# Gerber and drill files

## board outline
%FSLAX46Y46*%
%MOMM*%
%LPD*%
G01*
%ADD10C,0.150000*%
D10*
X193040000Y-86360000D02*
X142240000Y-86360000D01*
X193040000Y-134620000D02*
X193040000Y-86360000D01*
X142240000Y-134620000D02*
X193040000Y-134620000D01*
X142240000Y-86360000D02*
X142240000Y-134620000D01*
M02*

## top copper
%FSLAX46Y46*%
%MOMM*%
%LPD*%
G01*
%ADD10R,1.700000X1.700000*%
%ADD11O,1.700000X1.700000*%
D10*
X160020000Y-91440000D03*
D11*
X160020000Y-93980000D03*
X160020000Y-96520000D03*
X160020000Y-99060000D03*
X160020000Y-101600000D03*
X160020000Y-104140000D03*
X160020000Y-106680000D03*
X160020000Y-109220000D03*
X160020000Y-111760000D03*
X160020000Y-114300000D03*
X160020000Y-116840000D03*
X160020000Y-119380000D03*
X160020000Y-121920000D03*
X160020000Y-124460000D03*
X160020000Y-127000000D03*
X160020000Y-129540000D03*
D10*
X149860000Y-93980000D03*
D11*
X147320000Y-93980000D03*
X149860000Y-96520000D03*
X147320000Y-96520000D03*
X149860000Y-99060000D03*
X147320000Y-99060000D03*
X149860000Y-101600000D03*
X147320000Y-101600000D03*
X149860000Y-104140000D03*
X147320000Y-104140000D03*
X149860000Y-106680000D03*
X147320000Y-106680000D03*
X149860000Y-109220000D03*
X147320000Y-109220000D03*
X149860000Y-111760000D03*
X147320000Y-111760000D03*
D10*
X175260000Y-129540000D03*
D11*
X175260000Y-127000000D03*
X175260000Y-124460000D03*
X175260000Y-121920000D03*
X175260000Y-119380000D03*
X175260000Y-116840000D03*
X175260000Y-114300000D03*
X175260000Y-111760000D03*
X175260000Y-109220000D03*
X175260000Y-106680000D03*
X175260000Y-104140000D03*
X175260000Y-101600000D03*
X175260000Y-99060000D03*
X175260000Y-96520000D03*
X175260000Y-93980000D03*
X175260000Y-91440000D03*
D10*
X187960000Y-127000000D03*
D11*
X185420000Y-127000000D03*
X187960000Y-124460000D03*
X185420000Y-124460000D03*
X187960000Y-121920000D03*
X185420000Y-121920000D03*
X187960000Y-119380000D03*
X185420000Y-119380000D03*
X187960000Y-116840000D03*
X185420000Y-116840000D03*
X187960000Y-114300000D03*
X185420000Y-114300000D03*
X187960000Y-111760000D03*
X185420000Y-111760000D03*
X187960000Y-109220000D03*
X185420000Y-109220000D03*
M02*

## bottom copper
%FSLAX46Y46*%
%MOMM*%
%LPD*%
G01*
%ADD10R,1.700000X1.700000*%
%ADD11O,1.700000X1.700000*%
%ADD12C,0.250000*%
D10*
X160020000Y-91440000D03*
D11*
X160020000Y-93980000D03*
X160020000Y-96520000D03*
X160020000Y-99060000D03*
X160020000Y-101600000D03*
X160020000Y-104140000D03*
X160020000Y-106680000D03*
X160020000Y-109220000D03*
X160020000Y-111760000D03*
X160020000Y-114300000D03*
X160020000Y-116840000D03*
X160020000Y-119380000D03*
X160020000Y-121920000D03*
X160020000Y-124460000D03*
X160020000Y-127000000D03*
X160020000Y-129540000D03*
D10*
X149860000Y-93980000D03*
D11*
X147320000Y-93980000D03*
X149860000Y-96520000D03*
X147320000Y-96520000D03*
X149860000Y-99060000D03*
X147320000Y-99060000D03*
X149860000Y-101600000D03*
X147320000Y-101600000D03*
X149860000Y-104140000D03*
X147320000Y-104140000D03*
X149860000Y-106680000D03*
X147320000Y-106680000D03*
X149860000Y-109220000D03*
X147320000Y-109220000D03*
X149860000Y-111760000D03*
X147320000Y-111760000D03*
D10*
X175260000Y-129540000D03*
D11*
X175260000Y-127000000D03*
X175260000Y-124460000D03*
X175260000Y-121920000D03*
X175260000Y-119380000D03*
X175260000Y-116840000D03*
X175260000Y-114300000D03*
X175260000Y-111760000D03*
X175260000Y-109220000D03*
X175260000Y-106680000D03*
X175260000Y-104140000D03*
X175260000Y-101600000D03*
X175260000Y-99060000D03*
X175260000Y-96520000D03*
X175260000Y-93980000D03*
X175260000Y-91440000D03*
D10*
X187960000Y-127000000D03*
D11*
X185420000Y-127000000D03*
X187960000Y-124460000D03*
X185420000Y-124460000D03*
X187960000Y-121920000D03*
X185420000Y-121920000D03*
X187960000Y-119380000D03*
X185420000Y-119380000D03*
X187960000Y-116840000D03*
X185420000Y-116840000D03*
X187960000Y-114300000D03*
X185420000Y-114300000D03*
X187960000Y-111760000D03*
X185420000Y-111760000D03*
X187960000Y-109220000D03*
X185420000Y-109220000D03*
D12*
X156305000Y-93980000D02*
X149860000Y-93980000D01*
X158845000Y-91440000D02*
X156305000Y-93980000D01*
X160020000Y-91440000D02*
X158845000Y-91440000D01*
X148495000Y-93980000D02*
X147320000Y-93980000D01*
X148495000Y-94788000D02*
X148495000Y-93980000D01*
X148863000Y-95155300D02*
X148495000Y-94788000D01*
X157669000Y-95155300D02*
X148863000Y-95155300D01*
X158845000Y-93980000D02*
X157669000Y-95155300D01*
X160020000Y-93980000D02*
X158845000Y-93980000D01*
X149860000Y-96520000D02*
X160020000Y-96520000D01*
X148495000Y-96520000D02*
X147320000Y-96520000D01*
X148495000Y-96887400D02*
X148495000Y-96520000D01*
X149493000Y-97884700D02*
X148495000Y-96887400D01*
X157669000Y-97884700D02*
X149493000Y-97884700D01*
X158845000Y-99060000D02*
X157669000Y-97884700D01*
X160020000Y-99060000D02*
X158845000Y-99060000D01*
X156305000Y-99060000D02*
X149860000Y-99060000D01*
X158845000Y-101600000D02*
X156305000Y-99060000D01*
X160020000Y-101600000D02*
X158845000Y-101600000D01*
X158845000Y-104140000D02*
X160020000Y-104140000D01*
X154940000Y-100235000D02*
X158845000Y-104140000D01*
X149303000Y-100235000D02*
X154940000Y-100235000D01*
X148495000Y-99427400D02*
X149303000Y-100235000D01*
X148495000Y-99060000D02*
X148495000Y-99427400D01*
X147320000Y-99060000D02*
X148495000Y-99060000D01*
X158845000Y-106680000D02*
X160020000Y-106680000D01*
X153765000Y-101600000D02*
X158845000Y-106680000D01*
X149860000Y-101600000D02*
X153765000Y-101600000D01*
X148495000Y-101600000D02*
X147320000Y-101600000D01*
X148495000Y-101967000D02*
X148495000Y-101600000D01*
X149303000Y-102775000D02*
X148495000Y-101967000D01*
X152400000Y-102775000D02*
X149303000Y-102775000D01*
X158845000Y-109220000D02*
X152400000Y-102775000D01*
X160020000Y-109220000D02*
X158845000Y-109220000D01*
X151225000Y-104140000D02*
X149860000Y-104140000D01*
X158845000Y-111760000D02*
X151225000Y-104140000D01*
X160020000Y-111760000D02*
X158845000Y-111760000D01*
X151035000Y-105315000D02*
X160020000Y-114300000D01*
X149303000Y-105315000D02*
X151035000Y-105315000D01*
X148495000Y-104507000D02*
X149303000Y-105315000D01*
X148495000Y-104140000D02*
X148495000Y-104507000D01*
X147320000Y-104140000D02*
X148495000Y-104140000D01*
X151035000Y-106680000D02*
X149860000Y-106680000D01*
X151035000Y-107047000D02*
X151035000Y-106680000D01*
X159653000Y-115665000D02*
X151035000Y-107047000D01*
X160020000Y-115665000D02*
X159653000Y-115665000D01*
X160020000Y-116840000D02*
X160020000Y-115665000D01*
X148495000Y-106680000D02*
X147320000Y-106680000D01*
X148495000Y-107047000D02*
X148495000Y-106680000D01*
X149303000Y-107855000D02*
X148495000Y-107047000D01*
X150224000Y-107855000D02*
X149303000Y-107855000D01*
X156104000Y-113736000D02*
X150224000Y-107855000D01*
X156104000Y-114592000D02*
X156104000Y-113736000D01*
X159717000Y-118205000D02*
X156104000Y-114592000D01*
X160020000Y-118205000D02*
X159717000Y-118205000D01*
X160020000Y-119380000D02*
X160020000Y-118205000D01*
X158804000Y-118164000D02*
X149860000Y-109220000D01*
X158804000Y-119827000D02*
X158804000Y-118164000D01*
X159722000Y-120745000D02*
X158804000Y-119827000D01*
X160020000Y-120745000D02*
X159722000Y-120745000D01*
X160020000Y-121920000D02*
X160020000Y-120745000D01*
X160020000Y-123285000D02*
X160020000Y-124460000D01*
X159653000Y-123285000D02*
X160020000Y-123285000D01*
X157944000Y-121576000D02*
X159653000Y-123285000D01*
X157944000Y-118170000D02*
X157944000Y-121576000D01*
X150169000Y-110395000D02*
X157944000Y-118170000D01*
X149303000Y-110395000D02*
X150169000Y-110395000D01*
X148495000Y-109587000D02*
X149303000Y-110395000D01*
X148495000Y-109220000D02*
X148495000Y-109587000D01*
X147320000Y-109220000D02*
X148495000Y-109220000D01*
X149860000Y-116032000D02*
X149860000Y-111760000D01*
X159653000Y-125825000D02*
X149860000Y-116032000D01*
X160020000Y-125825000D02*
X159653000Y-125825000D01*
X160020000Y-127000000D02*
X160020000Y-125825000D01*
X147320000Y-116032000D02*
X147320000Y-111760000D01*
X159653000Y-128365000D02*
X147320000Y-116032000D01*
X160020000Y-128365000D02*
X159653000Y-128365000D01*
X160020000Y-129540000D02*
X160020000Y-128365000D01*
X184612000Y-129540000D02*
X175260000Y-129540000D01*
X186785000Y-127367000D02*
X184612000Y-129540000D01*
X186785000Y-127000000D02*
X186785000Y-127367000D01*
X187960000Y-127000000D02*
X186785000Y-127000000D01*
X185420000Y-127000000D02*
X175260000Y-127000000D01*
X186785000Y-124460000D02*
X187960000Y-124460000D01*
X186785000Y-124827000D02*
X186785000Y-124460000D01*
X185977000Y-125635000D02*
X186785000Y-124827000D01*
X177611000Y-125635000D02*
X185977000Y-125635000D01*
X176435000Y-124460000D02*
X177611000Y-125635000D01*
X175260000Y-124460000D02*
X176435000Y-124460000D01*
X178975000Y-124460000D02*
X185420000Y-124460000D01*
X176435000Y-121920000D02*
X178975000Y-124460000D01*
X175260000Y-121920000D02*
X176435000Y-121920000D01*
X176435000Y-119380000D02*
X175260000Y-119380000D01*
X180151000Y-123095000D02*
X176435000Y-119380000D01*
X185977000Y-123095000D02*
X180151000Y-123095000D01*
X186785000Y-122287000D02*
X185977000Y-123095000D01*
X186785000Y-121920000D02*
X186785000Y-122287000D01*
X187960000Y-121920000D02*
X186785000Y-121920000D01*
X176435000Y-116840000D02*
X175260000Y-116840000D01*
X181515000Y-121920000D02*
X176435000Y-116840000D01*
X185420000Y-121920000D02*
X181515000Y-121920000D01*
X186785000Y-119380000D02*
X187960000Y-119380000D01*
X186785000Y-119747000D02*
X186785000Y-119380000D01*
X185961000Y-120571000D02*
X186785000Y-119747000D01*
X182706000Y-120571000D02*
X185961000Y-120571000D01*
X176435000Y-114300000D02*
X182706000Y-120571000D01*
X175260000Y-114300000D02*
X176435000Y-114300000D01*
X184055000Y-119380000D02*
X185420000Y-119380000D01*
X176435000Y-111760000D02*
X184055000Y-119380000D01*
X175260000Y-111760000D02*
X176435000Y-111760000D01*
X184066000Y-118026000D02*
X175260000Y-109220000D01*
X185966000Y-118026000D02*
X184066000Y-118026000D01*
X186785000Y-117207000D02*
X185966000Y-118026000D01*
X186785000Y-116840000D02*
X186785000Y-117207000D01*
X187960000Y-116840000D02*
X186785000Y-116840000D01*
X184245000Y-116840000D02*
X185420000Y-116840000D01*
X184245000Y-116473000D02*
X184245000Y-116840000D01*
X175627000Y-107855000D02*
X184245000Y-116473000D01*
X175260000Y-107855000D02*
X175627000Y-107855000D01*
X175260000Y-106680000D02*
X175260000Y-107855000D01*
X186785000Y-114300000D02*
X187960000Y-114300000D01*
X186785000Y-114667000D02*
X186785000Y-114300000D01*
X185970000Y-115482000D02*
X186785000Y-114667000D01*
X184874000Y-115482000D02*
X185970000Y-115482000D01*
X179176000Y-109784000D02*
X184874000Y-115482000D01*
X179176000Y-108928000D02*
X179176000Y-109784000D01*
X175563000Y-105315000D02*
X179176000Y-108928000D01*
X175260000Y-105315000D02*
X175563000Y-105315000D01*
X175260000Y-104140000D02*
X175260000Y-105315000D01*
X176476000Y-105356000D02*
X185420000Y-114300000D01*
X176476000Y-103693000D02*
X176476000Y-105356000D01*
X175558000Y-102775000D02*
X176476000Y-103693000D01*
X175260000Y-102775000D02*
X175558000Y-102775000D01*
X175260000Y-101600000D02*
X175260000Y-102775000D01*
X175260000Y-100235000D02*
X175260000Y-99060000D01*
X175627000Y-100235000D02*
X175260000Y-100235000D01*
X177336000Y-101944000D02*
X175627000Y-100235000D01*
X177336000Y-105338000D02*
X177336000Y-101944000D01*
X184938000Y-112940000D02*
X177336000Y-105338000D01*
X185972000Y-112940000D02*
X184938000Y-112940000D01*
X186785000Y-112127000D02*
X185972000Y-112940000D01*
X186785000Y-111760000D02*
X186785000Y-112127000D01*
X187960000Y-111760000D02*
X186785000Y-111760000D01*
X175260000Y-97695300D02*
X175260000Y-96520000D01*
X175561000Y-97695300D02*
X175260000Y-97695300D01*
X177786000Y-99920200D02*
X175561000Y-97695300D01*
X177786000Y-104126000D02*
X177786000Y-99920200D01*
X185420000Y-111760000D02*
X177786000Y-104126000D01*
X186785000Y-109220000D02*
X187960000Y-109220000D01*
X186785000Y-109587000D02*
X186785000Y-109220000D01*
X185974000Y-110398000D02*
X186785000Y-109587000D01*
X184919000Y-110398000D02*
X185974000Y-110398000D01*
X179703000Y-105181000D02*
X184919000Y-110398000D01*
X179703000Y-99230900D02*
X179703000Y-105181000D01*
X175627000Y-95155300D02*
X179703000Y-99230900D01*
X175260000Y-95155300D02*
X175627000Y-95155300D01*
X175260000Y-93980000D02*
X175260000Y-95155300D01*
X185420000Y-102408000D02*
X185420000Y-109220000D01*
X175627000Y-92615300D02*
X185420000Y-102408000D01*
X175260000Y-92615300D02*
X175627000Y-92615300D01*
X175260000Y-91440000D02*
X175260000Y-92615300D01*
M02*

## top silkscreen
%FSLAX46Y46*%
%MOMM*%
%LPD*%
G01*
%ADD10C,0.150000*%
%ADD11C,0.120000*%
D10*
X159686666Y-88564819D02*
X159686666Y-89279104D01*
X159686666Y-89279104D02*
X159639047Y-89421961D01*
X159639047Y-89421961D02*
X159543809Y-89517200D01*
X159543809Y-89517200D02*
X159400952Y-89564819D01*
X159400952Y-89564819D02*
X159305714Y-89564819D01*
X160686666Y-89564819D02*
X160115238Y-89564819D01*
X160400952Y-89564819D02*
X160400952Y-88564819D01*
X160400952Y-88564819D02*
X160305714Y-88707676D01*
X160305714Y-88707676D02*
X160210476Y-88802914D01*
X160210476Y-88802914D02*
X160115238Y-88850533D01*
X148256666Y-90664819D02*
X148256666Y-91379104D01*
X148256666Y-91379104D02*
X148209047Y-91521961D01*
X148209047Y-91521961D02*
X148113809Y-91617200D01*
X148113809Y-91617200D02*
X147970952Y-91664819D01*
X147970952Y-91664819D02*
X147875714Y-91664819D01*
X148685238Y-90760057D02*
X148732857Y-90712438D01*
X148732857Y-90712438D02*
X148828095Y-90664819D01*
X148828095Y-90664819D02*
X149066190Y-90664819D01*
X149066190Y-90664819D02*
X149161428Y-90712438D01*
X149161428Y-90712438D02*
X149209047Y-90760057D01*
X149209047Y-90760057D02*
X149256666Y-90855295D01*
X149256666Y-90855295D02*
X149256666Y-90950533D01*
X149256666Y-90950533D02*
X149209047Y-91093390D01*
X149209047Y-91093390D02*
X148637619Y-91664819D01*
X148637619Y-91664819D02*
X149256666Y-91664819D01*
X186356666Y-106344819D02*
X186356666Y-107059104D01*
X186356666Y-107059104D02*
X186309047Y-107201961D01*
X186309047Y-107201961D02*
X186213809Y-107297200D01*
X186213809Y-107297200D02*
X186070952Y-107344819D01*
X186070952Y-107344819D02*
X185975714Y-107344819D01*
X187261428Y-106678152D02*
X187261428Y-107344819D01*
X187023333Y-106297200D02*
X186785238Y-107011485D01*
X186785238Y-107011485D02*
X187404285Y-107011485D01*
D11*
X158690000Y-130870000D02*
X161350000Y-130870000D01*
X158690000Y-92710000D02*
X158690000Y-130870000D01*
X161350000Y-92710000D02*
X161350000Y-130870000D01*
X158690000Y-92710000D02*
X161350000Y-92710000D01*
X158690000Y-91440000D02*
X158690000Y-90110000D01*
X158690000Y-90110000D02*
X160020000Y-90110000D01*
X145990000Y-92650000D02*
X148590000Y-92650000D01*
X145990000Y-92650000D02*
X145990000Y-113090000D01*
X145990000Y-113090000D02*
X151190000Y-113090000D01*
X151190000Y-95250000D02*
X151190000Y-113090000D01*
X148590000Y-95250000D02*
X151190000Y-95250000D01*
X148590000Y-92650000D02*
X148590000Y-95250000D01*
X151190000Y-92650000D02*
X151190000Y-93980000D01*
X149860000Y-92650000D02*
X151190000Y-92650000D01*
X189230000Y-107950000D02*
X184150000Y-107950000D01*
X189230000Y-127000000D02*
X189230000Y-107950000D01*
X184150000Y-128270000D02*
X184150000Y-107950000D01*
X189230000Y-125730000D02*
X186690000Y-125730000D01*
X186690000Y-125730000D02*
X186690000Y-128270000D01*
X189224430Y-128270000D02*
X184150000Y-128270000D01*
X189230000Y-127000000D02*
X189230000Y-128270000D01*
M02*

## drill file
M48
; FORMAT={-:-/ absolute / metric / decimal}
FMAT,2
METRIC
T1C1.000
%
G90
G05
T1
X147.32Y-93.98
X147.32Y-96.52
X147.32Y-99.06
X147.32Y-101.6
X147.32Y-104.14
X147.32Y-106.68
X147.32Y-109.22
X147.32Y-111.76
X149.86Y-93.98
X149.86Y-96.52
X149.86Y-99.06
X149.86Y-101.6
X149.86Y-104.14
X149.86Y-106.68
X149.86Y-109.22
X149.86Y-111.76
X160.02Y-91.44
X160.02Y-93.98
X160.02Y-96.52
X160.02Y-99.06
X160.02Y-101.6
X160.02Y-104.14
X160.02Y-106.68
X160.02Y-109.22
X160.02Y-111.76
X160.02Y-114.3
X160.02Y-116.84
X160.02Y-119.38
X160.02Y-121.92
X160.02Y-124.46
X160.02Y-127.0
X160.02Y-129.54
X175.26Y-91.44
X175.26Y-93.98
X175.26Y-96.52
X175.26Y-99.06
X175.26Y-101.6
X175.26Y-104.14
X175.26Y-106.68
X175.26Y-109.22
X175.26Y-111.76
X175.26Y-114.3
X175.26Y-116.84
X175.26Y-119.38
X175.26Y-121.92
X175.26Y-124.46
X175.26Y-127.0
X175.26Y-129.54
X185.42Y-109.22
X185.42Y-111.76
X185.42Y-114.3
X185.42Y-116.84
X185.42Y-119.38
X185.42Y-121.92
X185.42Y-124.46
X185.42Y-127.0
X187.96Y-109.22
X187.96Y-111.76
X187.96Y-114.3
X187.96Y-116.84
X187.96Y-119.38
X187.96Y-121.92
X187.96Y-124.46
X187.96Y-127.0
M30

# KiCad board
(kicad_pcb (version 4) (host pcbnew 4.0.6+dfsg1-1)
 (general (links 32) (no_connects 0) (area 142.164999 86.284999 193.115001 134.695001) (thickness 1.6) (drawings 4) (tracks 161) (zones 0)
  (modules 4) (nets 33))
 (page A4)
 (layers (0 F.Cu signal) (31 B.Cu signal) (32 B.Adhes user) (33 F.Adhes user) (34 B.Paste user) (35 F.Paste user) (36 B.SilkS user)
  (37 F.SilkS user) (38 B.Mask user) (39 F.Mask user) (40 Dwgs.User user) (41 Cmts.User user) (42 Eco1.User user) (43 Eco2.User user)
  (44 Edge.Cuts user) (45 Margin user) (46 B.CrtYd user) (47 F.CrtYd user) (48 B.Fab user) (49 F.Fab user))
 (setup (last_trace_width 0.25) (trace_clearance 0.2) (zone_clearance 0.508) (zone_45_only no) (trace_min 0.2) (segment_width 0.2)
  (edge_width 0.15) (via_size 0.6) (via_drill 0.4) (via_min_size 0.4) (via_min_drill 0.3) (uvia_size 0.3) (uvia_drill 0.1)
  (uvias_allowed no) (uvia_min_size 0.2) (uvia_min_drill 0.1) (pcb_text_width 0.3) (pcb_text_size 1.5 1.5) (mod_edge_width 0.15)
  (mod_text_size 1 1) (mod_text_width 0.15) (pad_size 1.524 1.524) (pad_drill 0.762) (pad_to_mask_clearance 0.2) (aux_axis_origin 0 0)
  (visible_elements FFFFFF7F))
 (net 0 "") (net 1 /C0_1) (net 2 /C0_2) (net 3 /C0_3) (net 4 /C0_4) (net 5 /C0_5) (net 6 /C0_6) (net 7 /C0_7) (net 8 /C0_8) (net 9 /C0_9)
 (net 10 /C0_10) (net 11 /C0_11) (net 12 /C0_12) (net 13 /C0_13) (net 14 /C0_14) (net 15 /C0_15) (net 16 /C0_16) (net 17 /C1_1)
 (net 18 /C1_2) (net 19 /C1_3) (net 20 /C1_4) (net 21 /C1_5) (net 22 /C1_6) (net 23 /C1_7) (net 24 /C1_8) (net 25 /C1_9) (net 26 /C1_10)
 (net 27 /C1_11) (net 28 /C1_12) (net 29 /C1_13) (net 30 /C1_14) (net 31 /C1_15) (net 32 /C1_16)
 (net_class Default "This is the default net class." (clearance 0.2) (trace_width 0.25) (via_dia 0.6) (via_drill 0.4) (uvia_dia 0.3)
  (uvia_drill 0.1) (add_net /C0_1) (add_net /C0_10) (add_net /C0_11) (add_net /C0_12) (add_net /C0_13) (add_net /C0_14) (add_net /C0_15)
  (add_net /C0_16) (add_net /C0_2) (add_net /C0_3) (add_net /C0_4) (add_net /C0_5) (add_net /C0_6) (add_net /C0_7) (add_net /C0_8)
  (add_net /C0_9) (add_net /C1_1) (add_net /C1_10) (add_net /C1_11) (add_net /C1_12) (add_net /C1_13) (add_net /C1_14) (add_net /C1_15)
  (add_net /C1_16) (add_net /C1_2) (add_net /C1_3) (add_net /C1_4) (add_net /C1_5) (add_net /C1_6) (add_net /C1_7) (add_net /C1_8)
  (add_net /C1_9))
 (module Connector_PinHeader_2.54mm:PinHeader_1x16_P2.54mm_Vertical (layer F.Cu) (at 160.02 91.44)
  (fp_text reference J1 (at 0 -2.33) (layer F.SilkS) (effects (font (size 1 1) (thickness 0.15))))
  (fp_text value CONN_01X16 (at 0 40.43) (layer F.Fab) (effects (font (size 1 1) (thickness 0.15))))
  (fp_line (start -1.33 39.43) (end 1.33 39.43) (layer F.SilkS) (width 0.12))
  (fp_line (start -1.33 1.27) (end -1.33 39.43) (layer F.SilkS) (width 0.12))
  (fp_line (start 1.33 1.27) (end 1.33 39.43) (layer F.SilkS) (width 0.12))
  (fp_line (start -1.33 1.27) (end 1.33 1.27) (layer F.SilkS) (width 0.12))
  (fp_line (start -1.33 0) (end -1.33 -1.33) (layer F.SilkS) (width 0.12))
  (fp_line (start -1.33 -1.33) (end 0 -1.33) (layer F.SilkS) (width 0.12))
  (pad 1 thru_hole rect (at 0 0) (size 1.7 1.7) (drill 1) (layers *.Cu *.Mask) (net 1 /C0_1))
  (pad 2 thru_hole oval (at 0 2.54) (size 1.7 1.7) (drill 1) (layers *.Cu *.Mask) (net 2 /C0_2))
  (pad 3 thru_hole oval (at 0 5.08) (size 1.7 1.7) (drill 1) (layers *.Cu *.Mask) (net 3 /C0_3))
  (pad 4 thru_hole oval (at 0 7.62) (size 1.7 1.7) (drill 1) (layers *.Cu *.Mask) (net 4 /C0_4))
  (pad 5 thru_hole oval (at 0 10.16) (size 1.7 1.7) (drill 1) (layers *.Cu *.Mask) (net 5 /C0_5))
  (pad 6 thru_hole oval (at 0 12.7) (size 1.7 1.7) (drill 1) (layers *.Cu *.Mask) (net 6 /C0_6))
  (pad 7 thru_hole oval (at 0 15.24) (size 1.7 1.7) (drill 1) (layers *.Cu *.Mask) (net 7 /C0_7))
  (pad 8 thru_hole oval (at 0 17.78) (size 1.7 1.7) (drill 1) (layers *.Cu *.Mask) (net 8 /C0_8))
  (pad 9 thru_hole oval (at 0 20.32) (size 1.7 1.7) (drill 1) (layers *.Cu *.Mask) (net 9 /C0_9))
  (pad 10 thru_hole oval (at 0 22.86) (size 1.7 1.7) (drill 1) (layers *.Cu *.Mask) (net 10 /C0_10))
  (pad 11 thru_hole oval (at 0 25.4) (size 1.7 1.7) (drill 1) (layers *.Cu *.Mask) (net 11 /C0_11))
  (pad 12 thru_hole oval (at 0 27.94) (size 1.7 1.7) (drill 1) (layers *.Cu *.Mask) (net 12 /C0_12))
  (pad 13 thru_hole oval (at 0 30.48) (size 1.7 1.7) (drill 1) (layers *.Cu *.Mask) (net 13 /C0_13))
  (pad 14 thru_hole oval (at 0 33.02) (size 1.7 1.7) (drill 1) (layers *.Cu *.Mask) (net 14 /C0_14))
  (pad 15 thru_hole oval (at 0 35.56) (size 1.7 1.7) (drill 1) (layers *.Cu *.Mask) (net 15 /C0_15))
  (pad 16 thru_hole oval (at 0 38.1) (size 1.7 1.7) (drill 1) (layers *.Cu *.Mask) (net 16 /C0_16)))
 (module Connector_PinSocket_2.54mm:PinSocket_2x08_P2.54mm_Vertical (layer F.Cu) (at 149.86 93.98)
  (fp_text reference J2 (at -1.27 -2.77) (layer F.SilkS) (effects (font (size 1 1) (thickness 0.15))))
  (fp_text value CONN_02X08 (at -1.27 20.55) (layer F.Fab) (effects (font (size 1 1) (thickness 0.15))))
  (fp_line (start -3.87 -1.33) (end -1.27 -1.33) (layer F.SilkS) (width 0.12))
  (fp_line (start -3.87 -1.33) (end -3.87 19.11) (layer F.SilkS) (width 0.12))
  (fp_line (start -3.87 19.11) (end 1.33 19.11) (layer F.SilkS) (width 0.12))
  (fp_line (start 1.33 1.27) (end 1.33 19.11) (layer F.SilkS) (width 0.12))
  (fp_line (start -1.27 1.27) (end 1.33 1.27) (layer F.SilkS) (width 0.12))
  (fp_line (start -1.27 -1.33) (end -1.27 1.27) (layer F.SilkS) (width 0.12))
  (fp_line (start 1.33 -1.33) (end 1.33 0) (layer F.SilkS) (width 0.12))
  (fp_line (start 0 -1.33) (end 1.33 -1.33) (layer F.SilkS) (width 0.12))
  (pad 1 thru_hole rect (at 0 0) (size 1.7 1.7) (drill 1) (layers *.Cu *.Mask) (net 1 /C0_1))
  (pad 2 thru_hole oval (at -2.54 0) (size 1.7 1.7) (drill 1) (layers *.Cu *.Mask) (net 2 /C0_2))
  (pad 3 thru_hole oval (at 0 2.54) (size 1.7 1.7) (drill 1) (layers *.Cu *.Mask) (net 3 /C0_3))
  (pad 4 thru_hole oval (at -2.54 2.54) (size 1.7 1.7) (drill 1) (layers *.Cu *.Mask) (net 4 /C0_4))
  (pad 5 thru_hole oval (at 0 5.08) (size 1.7 1.7) (drill 1) (layers *.Cu *.Mask) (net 5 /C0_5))
  (pad 6 thru_hole oval (at -2.54 5.08) (size 1.7 1.7) (drill 1) (layers *.Cu *.Mask) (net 6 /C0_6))
  (pad 7 thru_hole oval (at 0 7.62) (size 1.7 1.7) (drill 1) (layers *.Cu *.Mask) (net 7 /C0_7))
  (pad 8 thru_hole oval (at -2.54 7.62) (size 1.7 1.7) (drill 1) (layers *.Cu *.Mask) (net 8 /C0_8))
  (pad 9 thru_hole oval (at 0 10.16) (size 1.7 1.7) (drill 1) (layers *.Cu *.Mask) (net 9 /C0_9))
  (pad 10 thru_hole oval (at -2.54 10.16) (size 1.7 1.7) (drill 1) (layers *.Cu *.Mask) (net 10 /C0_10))
  (pad 11 thru_hole oval (at 0 12.7) (size 1.7 1.7) (drill 1) (layers *.Cu *.Mask) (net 11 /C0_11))
  (pad 12 thru_hole oval (at -2.54 12.7) (size 1.7 1.7) (drill 1) (layers *.Cu *.Mask) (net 12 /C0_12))
  (pad 13 thru_hole oval (at 0 15.24) (size 1.7 1.7) (drill 1) (layers *.Cu *.Mask) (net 13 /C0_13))
  (pad 14 thru_hole oval (at -2.54 15.24) (size 1.7 1.7) (drill 1) (layers *.Cu *.Mask) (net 14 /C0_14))
  (pad 15 thru_hole oval (at 0 17.78) (size 1.7 1.7) (drill 1) (layers *.Cu *.Mask) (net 15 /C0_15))
  (pad 16 thru_hole oval (at -2.54 17.78) (size 1.7 1.7) (drill 1) (layers *.Cu *.Mask) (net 16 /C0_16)))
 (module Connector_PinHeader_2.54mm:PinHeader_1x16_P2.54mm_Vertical (layer B.Cu) (at 175.26 129.54)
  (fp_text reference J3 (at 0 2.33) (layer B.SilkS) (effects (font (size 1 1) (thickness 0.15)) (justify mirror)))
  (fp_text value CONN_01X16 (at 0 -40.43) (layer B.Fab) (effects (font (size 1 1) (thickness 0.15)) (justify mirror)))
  (pad 1 thru_hole rect (at 0 0) (size 1.7 1.7) (drill 1) (layers *.Cu *.Mask) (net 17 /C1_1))
  (pad 2 thru_hole oval (at 0 -2.54) (size 1.7 1.7) (drill 1) (layers *.Cu *.Mask) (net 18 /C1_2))
  (pad 3 thru_hole oval (at 0 -5.08) (size 1.7 1.7) (drill 1) (layers *.Cu *.Mask) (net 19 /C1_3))
  (pad 4 thru_hole oval (at 0 -7.62) (size 1.7 1.7) (drill 1) (layers *.Cu *.Mask) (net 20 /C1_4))
  (pad 5 thru_hole oval (at 0 -10.16) (size 1.7 1.7) (drill 1) (layers *.Cu *.Mask) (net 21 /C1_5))
  (pad 6 thru_hole oval (at 0 -12.7) (size 1.7 1.7) (drill 1) (layers *.Cu *.Mask) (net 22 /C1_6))
  (pad 7 thru_hole oval (at 0 -15.24) (size 1.7 1.7) (drill 1) (layers *.Cu *.Mask) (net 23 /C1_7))
  (pad 8 thru_hole oval (at 0 -17.78) (size 1.7 1.7) (drill 1) (layers *.Cu *.Mask) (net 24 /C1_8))
  (pad 9 thru_hole oval (at 0 -20.32) (size 1.7 1.7) (drill 1) (layers *.Cu *.Mask) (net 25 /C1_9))
  (pad 10 thru_hole oval (at 0 -22.86) (size 1.7 1.7) (drill 1) (layers *.Cu *.Mask) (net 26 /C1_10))
  (pad 11 thru_hole oval (at 0 -25.4) (size 1.7 1.7) (drill 1) (layers *.Cu *.Mask) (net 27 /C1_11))
  (pad 12 thru_hole oval (at 0 -27.94) (size 1.7 1.7) (drill 1) (layers *.Cu *.Mask) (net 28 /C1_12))
  (pad 13 thru_hole oval (at 0 -30.48) (size 1.7 1.7) (drill 1) (layers *.Cu *.Mask) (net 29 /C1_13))
  (pad 14 thru_hole oval (at 0 -33.02) (size 1.7 1.7) (drill 1) (layers *.Cu *.Mask) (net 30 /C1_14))
  (pad 15 thru_hole oval (at 0 -35.56) (size 1.7 1.7) (drill 1) (layers *.Cu *.Mask) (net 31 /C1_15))
  (pad 16 thru_hole oval (at 0 -38.1) (size 1.7 1.7) (drill 1) (layers *.Cu *.Mask) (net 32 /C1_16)))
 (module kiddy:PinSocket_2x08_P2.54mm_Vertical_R (layer F.Cu) (at 187.96 127)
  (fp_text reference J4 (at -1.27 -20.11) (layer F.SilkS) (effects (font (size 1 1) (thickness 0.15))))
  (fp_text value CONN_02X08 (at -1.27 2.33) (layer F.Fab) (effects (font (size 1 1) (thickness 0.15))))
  (fp_line (start 1.27 -19.05) (end -3.81 -19.05) (layer F.SilkS) (width 0.12))
  (fp_line (start 1.27 0) (end 1.27 -19.05) (layer F.SilkS) (width 0.12))
  (fp_line (start -3.81 1.27) (end -3.81 -19.05) (layer F.SilkS) (width 0.12))
  (fp_line (start 1.27 -1.27) (end -1.27 -1.27) (layer F.SilkS) (width 0.12))
  (fp_line (start -1.27 -1.27) (end -1.27 1.27) (layer F.SilkS) (width 0.12))
  (fp_line (start 1.26443 1.27) (end -3.81 1.27) (layer F.SilkS) (width 0.12))
  (fp_line (start 1.27 0) (end 1.27 1.27) (layer F.SilkS) (width 0.12))
  (pad 1 thru_hole rect (at 0 0) (size 1.7 1.7) (drill 1) (layers *.Cu *.Mask) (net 17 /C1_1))
  (pad 2 thru_hole oval (at -2.54 0) (size 1.7 1.7) (drill 1) (layers *.Cu *.Mask) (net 18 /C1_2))
  (pad 3 thru_hole oval (at 0 -2.54) (size 1.7 1.7) (drill 1) (layers *.Cu *.Mask) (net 19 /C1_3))
  (pad 4 thru_hole oval (at -2.54 -2.54) (size 1.7 1.7) (drill 1) (layers *.Cu *.Mask) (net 20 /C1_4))
  (pad 5 thru_hole oval (at 0 -5.08) (size 1.7 1.7) (drill 1) (layers *.Cu *.Mask) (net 21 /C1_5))
  (pad 6 thru_hole oval (at -2.54 -5.08) (size 1.7 1.7) (drill 1) (layers *.Cu *.Mask) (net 22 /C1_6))
  (pad 7 thru_hole oval (at 0 -7.62) (size 1.7 1.7) (drill 1) (layers *.Cu *.Mask) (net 23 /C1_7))
  (pad 8 thru_hole oval (at -2.54 -7.62) (size 1.7 1.7) (drill 1) (layers *.Cu *.Mask) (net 24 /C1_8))
  (pad 9 thru_hole oval (at 0 -10.16) (size 1.7 1.7) (drill 1) (layers *.Cu *.Mask) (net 25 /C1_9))
  (pad 10 thru_hole oval (at -2.54 -10.16) (size 1.7 1.7) (drill 1) (layers *.Cu *.Mask) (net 26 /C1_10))
  (pad 11 thru_hole oval (at 0 -12.7) (size 1.7 1.7) (drill 1) (layers *.Cu *.Mask) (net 27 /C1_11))
  (pad 12 thru_hole oval (at -2.54 -12.7) (size 1.7 1.7) (drill 1) (layers *.Cu *.Mask) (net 28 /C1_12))
  (pad 13 thru_hole oval (at 0 -15.24) (size 1.7 1.7) (drill 1) (layers *.Cu *.Mask) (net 29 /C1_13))
  (pad 14 thru_hole oval (at -2.54 -15.24) (size 1.7 1.7) (drill 1) (layers *.Cu *.Mask) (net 30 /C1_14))
  (pad 15 thru_hole oval (at 0 -17.78) (size 1.7 1.7) (drill 1) (layers *.Cu *.Mask) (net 31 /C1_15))
  (pad 16 thru_hole oval (at -2.54 -17.78) (size 1.7 1.7) (drill 1) (layers *.Cu *.Mask) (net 32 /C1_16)))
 (gr_line (start 193.04 86.36) (end 142.24 86.36) (layer Edge.Cuts) (width 0.15))
 (gr_line (start 193.04 134.62) (end 193.04 86.36) (layer Edge.Cuts) (width 0.15))
 (gr_line (start 142.24 134.62) (end 193.04 134.62) (layer Edge.Cuts) (width 0.15))
 (gr_line (start 142.24 86.36) (end 142.24 134.62) (layer Edge.Cuts) (width 0.15))
 (segment (start 156.305 93.98) (end 149.86 93.98) (width 0.25) (layer B.Cu) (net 1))
 (segment (start 158.845 91.44) (end 156.305 93.98) (width 0.25) (layer B.Cu) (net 1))
 (segment (start 160.02 91.44) (end 158.845 91.44) (width 0.25) (layer B.Cu) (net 1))
 (segment (start 148.495 93.98) (end 147.32 93.98) (width 0.25) (layer B.Cu) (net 2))
 (segment (start 148.495 94.788) (end 148.495 93.98) (width 0.25) (layer B.Cu) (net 2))
 (segment (start 148.863 95.1553) (end 148.495 94.788) (width 0.25) (layer B.Cu) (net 2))
 (segment (start 157.669 95.1553) (end 148.863 95.1553) (width 0.25) (layer B.Cu) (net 2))
 (segment (start 158.845 93.98) (end 157.669 95.1553) (width 0.25) (layer B.Cu) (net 2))
 (segment (start 160.02 93.98) (end 158.845 93.98) (width 0.25) (layer B.Cu) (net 2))
 (segment (start 149.86 96.52) (end 160.02 96.52) (width 0.25) (layer B.Cu) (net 3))
 (segment (start 148.495 96.52) (end 147.32 96.52) (width 0.25) (layer B.Cu) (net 4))
 (segment (start 148.495 96.8874) (end 148.495 96.52) (width 0.25) (layer B.Cu) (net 4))
 (segment (start 149.493 97.8847) (end 148.495 96.8874) (width 0.25) (layer B.Cu) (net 4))
 (segment (start 157.669 97.8847) (end 149.493 97.8847) (width 0.25) (layer B.Cu) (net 4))
 (segment (start 158.845 99.06) (end 157.669 97.8847) (width 0.25) (layer B.Cu) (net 4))
 (segment (start 160.02 99.06) (end 158.845 99.06) (width 0.25) (layer B.Cu) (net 4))
 (segment (start 156.305 99.06) (end 149.86 99.06) (width 0.25) (layer B.Cu) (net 5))
 (segment (start 158.845 101.6) (end 156.305 99.06) (width 0.25) (layer B.Cu) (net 5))
 (segment (start 160.02 101.6) (end 158.845 101.6) (width 0.25) (layer B.Cu) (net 5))
 (segment (start 158.845 104.14) (end 160.02 104.14) (width 0.25) (layer B.Cu) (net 6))
 (segment (start 154.94 100.235) (end 158.845 104.14) (width 0.25) (layer B.Cu) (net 6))
 (segment (start 149.303 100.235) (end 154.94 100.235) (width 0.25) (layer B.Cu) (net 6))
 (segment (start 148.495 99.4274) (end 149.303 100.235) (width 0.25) (layer B.Cu) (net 6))
 (segment (start 148.495 99.06) (end 148.495 99.4274) (width 0.25) (layer B.Cu) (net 6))
 (segment (start 147.32 99.06) (end 148.495 99.06) (width 0.25) (layer B.Cu) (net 6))
 (segment (start 158.845 106.68) (end 160.02 106.68) (width 0.25) (layer B.Cu) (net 7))
 (segment (start 153.765 101.6) (end 158.845 106.68) (width 0.25) (layer B.Cu) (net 7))
 (segment (start 149.86 101.6) (end 153.765 101.6) (width 0.25) (layer B.Cu) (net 7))
 (segment (start 148.495 101.6) (end 147.32 101.6) (width 0.25) (layer B.Cu) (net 8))
 (segment (start 148.495 101.967) (end 148.495 101.6) (width 0.25) (layer B.Cu) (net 8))
 (segment (start 149.303 102.775) (end 148.495 101.967) (width 0.25) (layer B.Cu) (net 8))
 (segment (start 152.4 102.775) (end 149.303 102.775) (width 0.25) (layer B.Cu) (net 8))
 (segment (start 158.845 109.22) (end 152.4 102.775) (width 0.25) (layer B.Cu) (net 8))
 (segment (start 160.02 109.22) (end 158.845 109.22) (width 0.25) (layer B.Cu) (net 8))
 (segment (start 151.225 104.14) (end 149.86 104.14) (width 0.25) (layer B.Cu) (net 9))
 (segment (start 158.845 111.76) (end 151.225 104.14) (width 0.25) (layer B.Cu) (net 9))
 (segment (start 160.02 111.76) (end 158.845 111.76) (width 0.25) (layer B.Cu) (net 9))
 (segment (start 151.035 105.315) (end 160.02 114.3) (width 0.25) (layer B.Cu) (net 10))
 (segment (start 149.303 105.315) (end 151.035 105.315) (width 0.25) (layer B.Cu) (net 10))
 (segment (start 148.495 104.507) (end 149.303 105.315) (width 0.25) (layer B.Cu) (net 10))
 (segment (start 148.495 104.14) (end 148.495 104.507) (width 0.25) (layer B.Cu) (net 10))
 (segment (start 147.32 104.14) (end 148.495 104.14) (width 0.25) (layer B.Cu) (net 10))
 (segment (start 151.035 106.68) (end 149.86 106.68) (width 0.25) (layer B.Cu) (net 11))
 (segment (start 151.035 107.047) (end 151.035 106.68) (width 0.25) (layer B.Cu) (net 11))
 (segment (start 159.653 115.665) (end 151.035 107.047) (width 0.25) (layer B.Cu) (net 11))
 (segment (start 160.02 115.665) (end 159.653 115.665) (width 0.25) (layer B.Cu) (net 11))
 (segment (start 160.02 116.84) (end 160.02 115.665) (width 0.25) (layer B.Cu) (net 11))
 (segment (start 148.495 106.68) (end 147.32 106.68) (width 0.25) (layer B.Cu) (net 12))
 (segment (start 148.495 107.047) (end 148.495 106.68) (width 0.25) (layer B.Cu) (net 12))
 (segment (start 149.303 107.855) (end 148.495 107.047) (width 0.25) (layer B.Cu) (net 12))
 (segment (start 150.224 107.855) (end 149.303 107.855) (width 0.25) (layer B.Cu) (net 12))
 (segment (start 156.104 113.736) (end 150.224 107.855) (width 0.25) (layer B.Cu) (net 12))
 (segment (start 156.104 114.592) (end 156.104 113.736) (width 0.25) (layer B.Cu) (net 12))
 (segment (start 159.717 118.205) (end 156.104 114.592) (width 0.25) (layer B.Cu) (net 12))
 (segment (start 160.02 118.205) (end 159.717 118.205) (width 0.25) (layer B.Cu) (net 12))
 (segment (start 160.02 119.38) (end 160.02 118.205) (width 0.25) (layer B.Cu) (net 12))
 (segment (start 158.804 118.164) (end 149.86 109.22) (width 0.25) (layer B.Cu) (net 13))
 (segment (start 158.804 119.827) (end 158.804 118.164) (width 0.25) (layer B.Cu) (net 13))
 (segment (start 159.722 120.745) (end 158.804 119.827) (width 0.25) (layer B.Cu) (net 13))
 (segment (start 160.02 120.745) (end 159.722 120.745) (width 0.25) (layer B.Cu) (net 13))
 (segment (start 160.02 121.92) (end 160.02 120.745) (width 0.25) (layer B.Cu) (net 13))
 (segment (start 160.02 123.285) (end 160.02 124.46) (width 0.25) (layer B.Cu) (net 14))
 (segment (start 159.653 123.285) (end 160.02 123.285) (width 0.25) (layer B.Cu) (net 14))
 (segment (start 157.944 121.576) (end 159.653 123.285) (width 0.25) (layer B.Cu) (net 14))
 (segment (start 157.944 118.17) (end 157.944 121.576) (width 0.25) (layer B.Cu) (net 14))
 (segment (start 150.169 110.395) (end 157.944 118.17) (width 0.25) (layer B.Cu) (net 14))
 (segment (start 149.303 110.395) (end 150.169 110.395) (width 0.25) (layer B.Cu) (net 14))
 (segment (start 148.495 109.587) (end 149.303 110.395) (width 0.25) (layer B.Cu) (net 14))
 (segment (start 148.495 109.22) (end 148.495 109.587) (width 0.25) (layer B.Cu) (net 14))
 (segment (start 147.32 109.22) (end 148.495 109.22) (width 0.25) (layer B.Cu) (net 14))
 (segment (start 149.86 116.032) (end 149.86 111.76) (width 0.25) (layer B.Cu) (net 15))
 (segment (start 159.653 125.825) (end 149.86 116.032) (width 0.25) (layer B.Cu) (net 15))
 (segment (start 160.02 125.825) (end 159.653 125.825) (width 0.25) (layer B.Cu) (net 15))
 (segment (start 160.02 127) (end 160.02 125.825) (width 0.25) (layer B.Cu) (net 15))
 (segment (start 147.32 116.032) (end 147.32 111.76) (width 0.25) (layer B.Cu) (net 16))
 (segment (start 159.653 128.365) (end 147.32 116.032) (width 0.25) (layer B.Cu) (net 16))
 (segment (start 160.02 128.365) (end 159.653 128.365) (width 0.25) (layer B.Cu) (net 16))
 (segment (start 160.02 129.54) (end 160.02 128.365) (width 0.25) (layer B.Cu) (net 16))
 (segment (start 184.612 129.54) (end 175.26 129.54) (width 0.25) (layer B.Cu) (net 17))
 (segment (start 186.785 127.367) (end 184.612 129.54) (width 0.25) (layer B.Cu) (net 17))
 (segment (start 186.785 127) (end 186.785 127.367) (width 0.25) (layer B.Cu) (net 17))
 (segment (start 187.96 127) (end 186.785 127) (width 0.25) (layer B.Cu) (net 17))
 (segment (start 185.42 127) (end 175.26 127) (width 0.25) (layer B.Cu) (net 18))
 (segment (start 186.785 124.46) (end 187.96 124.46) (width 0.25) (layer B.Cu) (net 19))
 (segment (start 186.785 124.827) (end 186.785 124.46) (width 0.25) (layer B.Cu) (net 19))
 (segment (start 185.977 125.635) (end 186.785 124.827) (width 0.25) (layer B.Cu) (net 19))
 (segment (start 177.611 125.635) (end 185.977 125.635) (width 0.25) (layer B.Cu) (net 19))
 (segment (start 176.435 124.46) (end 177.611 125.635) (width 0.25) (layer B.Cu) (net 19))
 (segment (start 175.26 124.46) (end 176.435 124.46) (width 0.25) (layer B.Cu) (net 19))
 (segment (start 178.975 124.46) (end 185.42 124.46) (width 0.25) (layer B.Cu) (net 20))
 (segment (start 176.435 121.92) (end 178.975 124.46) (width 0.25) (layer B.Cu) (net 20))
 (segment (start 175.26 121.92) (end 176.435 121.92) (width 0.25) (layer B.Cu) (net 20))
 (segment (start 176.435 119.38) (end 175.26 119.38) (width 0.25) (layer B.Cu) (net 21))
 (segment (start 180.151 123.095) (end 176.435 119.38) (width 0.25) (layer B.Cu) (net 21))
 (segment (start 185.977 123.095) (end 180.151 123.095) (width 0.25) (layer B.Cu) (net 21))
 (segment (start 186.785 122.287) (end 185.977 123.095) (width 0.25) (layer B.Cu) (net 21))
 (segment (start 186.785 121.92) (end 186.785 122.287) (width 0.25) (layer B.Cu) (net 21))
 (segment (start 187.96 121.92) (end 186.785 121.92) (width 0.25) (layer B.Cu) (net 21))
 (segment (start 176.435 116.84) (end 175.26 116.84) (width 0.25) (layer B.Cu) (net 22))
 (segment (start 181.515 121.92) (end 176.435 116.84) (width 0.25) (layer B.Cu) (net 22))
 (segment (start 185.42 121.92) (end 181.515 121.92) (width 0.25) (layer B.Cu) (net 22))
 (segment (start 186.785 119.38) (end 187.96 119.38) (width 0.25) (layer B.Cu) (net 23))
 (segment (start 186.785 119.747) (end 186.785 119.38) (width 0.25) (layer B.Cu) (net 23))
 (segment (start 185.961 120.571) (end 186.785 119.747) (width 0.25) (layer B.Cu) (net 23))
 (segment (start 182.706 120.571) (end 185.961 120.571) (width 0.25) (layer B.Cu) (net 23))
 (segment (start 176.435 114.3) (end 182.706 120.571) (width 0.25) (layer B.Cu) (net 23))
 (segment (start 175.26 114.3) (end 176.435 114.3) (width 0.25) (layer B.Cu) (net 23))
 (segment (start 184.055 119.38) (end 185.42 119.38) (width 0.25) (layer B.Cu) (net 24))
 (segment (start 176.435 111.76) (end 184.055 119.38) (width 0.25) (layer B.Cu) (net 24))
 (segment (start 175.26 111.76) (end 176.435 111.76) (width 0.25) (layer B.Cu) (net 24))
 (segment (start 184.066 118.026) (end 175.26 109.22) (width 0.25) (layer B.Cu) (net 25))
 (segment (start 185.966 118.026) (end 184.066 118.026) (width 0.25) (layer B.Cu) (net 25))
 (segment (start 186.785 117.207) (end 185.966 118.026) (width 0.25) (layer B.Cu) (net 25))
 (segment (start 186.785 116.84) (end 186.785 117.207) (width 0.25) (layer B.Cu) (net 25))
 (segment (start 187.96 116.84) (end 186.785 116.84) (width 0.25) (layer B.Cu) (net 25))
 (segment (start 184.245 116.84) (end 185.42 116.84) (width 0.25) (layer B.Cu) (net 26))
 (segment (start 184.245 116.473) (end 184.245 116.84) (width 0.25) (layer B.Cu) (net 26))
 (segment (start 175.627 107.855) (end 184.245 116.473) (width 0.25) (layer B.Cu) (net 26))
 (segment (start 175.26 107.855) (end 175.627 107.855) (width 0.25) (layer B.Cu) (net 26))
 (segment (start 175.26 106.68) (end 175.26 107.855) (width 0.25) (layer B.Cu) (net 26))
 (segment (start 186.785 114.3) (end 187.96 114.3) (width 0.25) (layer B.Cu) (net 27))
 (segment (start 186.785 114.667) (end 186.785 114.3) (width 0.25) (layer B.Cu) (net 27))
 (segment (start 185.97 115.482) (end 186.785 114.667) (width 0.25) (layer B.Cu) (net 27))
 (segment (start 184.874 115.482) (end 185.97 115.482) (width 0.25) (layer B.Cu) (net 27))
 (segment (start 179.176 109.784) (end 184.874 115.482) (width 0.25) (layer B.Cu) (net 27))
 (segment (start 179.176 108.928) (end 179.176 109.784) (width 0.25) (layer B.Cu) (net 27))
 (segment (start 175.563 105.315) (end 179.176 108.928) (width 0.25) (layer B.Cu) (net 27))
 (segment (start 175.26 105.315) (end 175.563 105.315) (width 0.25) (layer B.Cu) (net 27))
 (segment (start 175.26 104.14) (end 175.26 105.315) (width 0.25) (layer B.Cu) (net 27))
 (segment (start 176.476 105.356) (end 185.42 114.3) (width 0.25) (layer B.Cu) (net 28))
 (segment (start 176.476 103.693) (end 176.476 105.356) (width 0.25) (layer B.Cu) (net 28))
 (segment (start 175.558 102.775) (end 176.476 103.693) (width 0.25) (layer B.Cu) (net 28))
 (segment (start 175.26 102.775) (end 175.558 102.775) (width 0.25) (layer B.Cu) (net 28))
 (segment (start 175.26 101.6) (end 175.26 102.775) (width 0.25) (layer B.Cu) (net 28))
 (segment (start 175.26 100.235) (end 175.26 99.06) (width 0.25) (layer B.Cu) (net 29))
 (segment (start 175.627 100.235) (end 175.26 100.235) (width 0.25) (layer B.Cu) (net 29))
 (segment (start 177.336 101.944) (end 175.627 100.235) (width 0.25) (layer B.Cu) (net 29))
 (segment (start 177.336 105.338) (end 177.336 101.944) (width 0.25) (layer B.Cu) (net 29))
 (segment (start 184.938 112.94) (end 177.336 105.338) (width 0.25) (layer B.Cu) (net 29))
 (segment (start 185.972 112.94) (end 184.938 112.94) (width 0.25) (layer B.Cu) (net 29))
 (segment (start 186.785 112.127) (end 185.972 112.94) (width 0.25) (layer B.Cu) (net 29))
 (segment (start 186.785 111.76) (end 186.785 112.127) (width 0.25) (layer B.Cu) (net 29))
 (segment (start 187.96 111.76) (end 186.785 111.76) (width 0.25) (layer B.Cu) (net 29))
 (segment (start 175.26 97.6953) (end 175.26 96.52) (width 0.25) (layer B.Cu) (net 30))
 (segment (start 175.561 97.6953) (end 175.26 97.6953) (width 0.25) (layer B.Cu) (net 30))
 (segment (start 177.786 99.9202) (end 175.561 97.6953) (width 0.25) (layer B.Cu) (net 30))
 (segment (start 177.786 104.126) (end 177.786 99.9202) (width 0.25) (layer B.Cu) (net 30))
 (segment (start 185.42 111.76) (end 177.786 104.126) (width 0.25) (layer B.Cu) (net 30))
 (segment (start 186.785 109.22) (end 187.96 109.22) (width 0.25) (layer B.Cu) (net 31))
 (segment (start 186.785 109.587) (end 186.785 109.22) (width 0.25) (layer B.Cu) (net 31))
 (segment (start 185.974 110.398) (end 186.785 109.587) (width 0.25) (layer B.Cu) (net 31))
 (segment (start 184.919 110.398) (end 185.974 110.398) (width 0.25) (layer B.Cu) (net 31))
 (segment (start 179.703 105.181) (end 184.919 110.398) (width 0.25) (layer B.Cu) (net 31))
 (segment (start 179.703 99.2309) (end 179.703 105.181) (width 0.25) (layer B.Cu) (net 31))
 (segment (start 175.627 95.1553) (end 179.703 99.2309) (width 0.25) (layer B.Cu) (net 31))
 (segment (start 175.26 95.1553) (end 175.627 95.1553) (width 0.25) (layer B.Cu) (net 31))
 (segment (start 175.26 93.98) (end 175.26 95.1553) (width 0.25) (layer B.Cu) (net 31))
 (segment (start 185.42 102.408) (end 185.42 109.22) (width 0.25) (layer B.Cu) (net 32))
 (segment (start 175.627 92.6153) (end 185.42 102.408) (width 0.25) (layer B.Cu) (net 32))
 (segment (start 175.26 92.6153) (end 175.627 92.6153) (width 0.25) (layer B.Cu) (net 32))
 (segment (start 175.26 91.44) (end 175.26 92.6153) (width 0.25) (layer B.Cu) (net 32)))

